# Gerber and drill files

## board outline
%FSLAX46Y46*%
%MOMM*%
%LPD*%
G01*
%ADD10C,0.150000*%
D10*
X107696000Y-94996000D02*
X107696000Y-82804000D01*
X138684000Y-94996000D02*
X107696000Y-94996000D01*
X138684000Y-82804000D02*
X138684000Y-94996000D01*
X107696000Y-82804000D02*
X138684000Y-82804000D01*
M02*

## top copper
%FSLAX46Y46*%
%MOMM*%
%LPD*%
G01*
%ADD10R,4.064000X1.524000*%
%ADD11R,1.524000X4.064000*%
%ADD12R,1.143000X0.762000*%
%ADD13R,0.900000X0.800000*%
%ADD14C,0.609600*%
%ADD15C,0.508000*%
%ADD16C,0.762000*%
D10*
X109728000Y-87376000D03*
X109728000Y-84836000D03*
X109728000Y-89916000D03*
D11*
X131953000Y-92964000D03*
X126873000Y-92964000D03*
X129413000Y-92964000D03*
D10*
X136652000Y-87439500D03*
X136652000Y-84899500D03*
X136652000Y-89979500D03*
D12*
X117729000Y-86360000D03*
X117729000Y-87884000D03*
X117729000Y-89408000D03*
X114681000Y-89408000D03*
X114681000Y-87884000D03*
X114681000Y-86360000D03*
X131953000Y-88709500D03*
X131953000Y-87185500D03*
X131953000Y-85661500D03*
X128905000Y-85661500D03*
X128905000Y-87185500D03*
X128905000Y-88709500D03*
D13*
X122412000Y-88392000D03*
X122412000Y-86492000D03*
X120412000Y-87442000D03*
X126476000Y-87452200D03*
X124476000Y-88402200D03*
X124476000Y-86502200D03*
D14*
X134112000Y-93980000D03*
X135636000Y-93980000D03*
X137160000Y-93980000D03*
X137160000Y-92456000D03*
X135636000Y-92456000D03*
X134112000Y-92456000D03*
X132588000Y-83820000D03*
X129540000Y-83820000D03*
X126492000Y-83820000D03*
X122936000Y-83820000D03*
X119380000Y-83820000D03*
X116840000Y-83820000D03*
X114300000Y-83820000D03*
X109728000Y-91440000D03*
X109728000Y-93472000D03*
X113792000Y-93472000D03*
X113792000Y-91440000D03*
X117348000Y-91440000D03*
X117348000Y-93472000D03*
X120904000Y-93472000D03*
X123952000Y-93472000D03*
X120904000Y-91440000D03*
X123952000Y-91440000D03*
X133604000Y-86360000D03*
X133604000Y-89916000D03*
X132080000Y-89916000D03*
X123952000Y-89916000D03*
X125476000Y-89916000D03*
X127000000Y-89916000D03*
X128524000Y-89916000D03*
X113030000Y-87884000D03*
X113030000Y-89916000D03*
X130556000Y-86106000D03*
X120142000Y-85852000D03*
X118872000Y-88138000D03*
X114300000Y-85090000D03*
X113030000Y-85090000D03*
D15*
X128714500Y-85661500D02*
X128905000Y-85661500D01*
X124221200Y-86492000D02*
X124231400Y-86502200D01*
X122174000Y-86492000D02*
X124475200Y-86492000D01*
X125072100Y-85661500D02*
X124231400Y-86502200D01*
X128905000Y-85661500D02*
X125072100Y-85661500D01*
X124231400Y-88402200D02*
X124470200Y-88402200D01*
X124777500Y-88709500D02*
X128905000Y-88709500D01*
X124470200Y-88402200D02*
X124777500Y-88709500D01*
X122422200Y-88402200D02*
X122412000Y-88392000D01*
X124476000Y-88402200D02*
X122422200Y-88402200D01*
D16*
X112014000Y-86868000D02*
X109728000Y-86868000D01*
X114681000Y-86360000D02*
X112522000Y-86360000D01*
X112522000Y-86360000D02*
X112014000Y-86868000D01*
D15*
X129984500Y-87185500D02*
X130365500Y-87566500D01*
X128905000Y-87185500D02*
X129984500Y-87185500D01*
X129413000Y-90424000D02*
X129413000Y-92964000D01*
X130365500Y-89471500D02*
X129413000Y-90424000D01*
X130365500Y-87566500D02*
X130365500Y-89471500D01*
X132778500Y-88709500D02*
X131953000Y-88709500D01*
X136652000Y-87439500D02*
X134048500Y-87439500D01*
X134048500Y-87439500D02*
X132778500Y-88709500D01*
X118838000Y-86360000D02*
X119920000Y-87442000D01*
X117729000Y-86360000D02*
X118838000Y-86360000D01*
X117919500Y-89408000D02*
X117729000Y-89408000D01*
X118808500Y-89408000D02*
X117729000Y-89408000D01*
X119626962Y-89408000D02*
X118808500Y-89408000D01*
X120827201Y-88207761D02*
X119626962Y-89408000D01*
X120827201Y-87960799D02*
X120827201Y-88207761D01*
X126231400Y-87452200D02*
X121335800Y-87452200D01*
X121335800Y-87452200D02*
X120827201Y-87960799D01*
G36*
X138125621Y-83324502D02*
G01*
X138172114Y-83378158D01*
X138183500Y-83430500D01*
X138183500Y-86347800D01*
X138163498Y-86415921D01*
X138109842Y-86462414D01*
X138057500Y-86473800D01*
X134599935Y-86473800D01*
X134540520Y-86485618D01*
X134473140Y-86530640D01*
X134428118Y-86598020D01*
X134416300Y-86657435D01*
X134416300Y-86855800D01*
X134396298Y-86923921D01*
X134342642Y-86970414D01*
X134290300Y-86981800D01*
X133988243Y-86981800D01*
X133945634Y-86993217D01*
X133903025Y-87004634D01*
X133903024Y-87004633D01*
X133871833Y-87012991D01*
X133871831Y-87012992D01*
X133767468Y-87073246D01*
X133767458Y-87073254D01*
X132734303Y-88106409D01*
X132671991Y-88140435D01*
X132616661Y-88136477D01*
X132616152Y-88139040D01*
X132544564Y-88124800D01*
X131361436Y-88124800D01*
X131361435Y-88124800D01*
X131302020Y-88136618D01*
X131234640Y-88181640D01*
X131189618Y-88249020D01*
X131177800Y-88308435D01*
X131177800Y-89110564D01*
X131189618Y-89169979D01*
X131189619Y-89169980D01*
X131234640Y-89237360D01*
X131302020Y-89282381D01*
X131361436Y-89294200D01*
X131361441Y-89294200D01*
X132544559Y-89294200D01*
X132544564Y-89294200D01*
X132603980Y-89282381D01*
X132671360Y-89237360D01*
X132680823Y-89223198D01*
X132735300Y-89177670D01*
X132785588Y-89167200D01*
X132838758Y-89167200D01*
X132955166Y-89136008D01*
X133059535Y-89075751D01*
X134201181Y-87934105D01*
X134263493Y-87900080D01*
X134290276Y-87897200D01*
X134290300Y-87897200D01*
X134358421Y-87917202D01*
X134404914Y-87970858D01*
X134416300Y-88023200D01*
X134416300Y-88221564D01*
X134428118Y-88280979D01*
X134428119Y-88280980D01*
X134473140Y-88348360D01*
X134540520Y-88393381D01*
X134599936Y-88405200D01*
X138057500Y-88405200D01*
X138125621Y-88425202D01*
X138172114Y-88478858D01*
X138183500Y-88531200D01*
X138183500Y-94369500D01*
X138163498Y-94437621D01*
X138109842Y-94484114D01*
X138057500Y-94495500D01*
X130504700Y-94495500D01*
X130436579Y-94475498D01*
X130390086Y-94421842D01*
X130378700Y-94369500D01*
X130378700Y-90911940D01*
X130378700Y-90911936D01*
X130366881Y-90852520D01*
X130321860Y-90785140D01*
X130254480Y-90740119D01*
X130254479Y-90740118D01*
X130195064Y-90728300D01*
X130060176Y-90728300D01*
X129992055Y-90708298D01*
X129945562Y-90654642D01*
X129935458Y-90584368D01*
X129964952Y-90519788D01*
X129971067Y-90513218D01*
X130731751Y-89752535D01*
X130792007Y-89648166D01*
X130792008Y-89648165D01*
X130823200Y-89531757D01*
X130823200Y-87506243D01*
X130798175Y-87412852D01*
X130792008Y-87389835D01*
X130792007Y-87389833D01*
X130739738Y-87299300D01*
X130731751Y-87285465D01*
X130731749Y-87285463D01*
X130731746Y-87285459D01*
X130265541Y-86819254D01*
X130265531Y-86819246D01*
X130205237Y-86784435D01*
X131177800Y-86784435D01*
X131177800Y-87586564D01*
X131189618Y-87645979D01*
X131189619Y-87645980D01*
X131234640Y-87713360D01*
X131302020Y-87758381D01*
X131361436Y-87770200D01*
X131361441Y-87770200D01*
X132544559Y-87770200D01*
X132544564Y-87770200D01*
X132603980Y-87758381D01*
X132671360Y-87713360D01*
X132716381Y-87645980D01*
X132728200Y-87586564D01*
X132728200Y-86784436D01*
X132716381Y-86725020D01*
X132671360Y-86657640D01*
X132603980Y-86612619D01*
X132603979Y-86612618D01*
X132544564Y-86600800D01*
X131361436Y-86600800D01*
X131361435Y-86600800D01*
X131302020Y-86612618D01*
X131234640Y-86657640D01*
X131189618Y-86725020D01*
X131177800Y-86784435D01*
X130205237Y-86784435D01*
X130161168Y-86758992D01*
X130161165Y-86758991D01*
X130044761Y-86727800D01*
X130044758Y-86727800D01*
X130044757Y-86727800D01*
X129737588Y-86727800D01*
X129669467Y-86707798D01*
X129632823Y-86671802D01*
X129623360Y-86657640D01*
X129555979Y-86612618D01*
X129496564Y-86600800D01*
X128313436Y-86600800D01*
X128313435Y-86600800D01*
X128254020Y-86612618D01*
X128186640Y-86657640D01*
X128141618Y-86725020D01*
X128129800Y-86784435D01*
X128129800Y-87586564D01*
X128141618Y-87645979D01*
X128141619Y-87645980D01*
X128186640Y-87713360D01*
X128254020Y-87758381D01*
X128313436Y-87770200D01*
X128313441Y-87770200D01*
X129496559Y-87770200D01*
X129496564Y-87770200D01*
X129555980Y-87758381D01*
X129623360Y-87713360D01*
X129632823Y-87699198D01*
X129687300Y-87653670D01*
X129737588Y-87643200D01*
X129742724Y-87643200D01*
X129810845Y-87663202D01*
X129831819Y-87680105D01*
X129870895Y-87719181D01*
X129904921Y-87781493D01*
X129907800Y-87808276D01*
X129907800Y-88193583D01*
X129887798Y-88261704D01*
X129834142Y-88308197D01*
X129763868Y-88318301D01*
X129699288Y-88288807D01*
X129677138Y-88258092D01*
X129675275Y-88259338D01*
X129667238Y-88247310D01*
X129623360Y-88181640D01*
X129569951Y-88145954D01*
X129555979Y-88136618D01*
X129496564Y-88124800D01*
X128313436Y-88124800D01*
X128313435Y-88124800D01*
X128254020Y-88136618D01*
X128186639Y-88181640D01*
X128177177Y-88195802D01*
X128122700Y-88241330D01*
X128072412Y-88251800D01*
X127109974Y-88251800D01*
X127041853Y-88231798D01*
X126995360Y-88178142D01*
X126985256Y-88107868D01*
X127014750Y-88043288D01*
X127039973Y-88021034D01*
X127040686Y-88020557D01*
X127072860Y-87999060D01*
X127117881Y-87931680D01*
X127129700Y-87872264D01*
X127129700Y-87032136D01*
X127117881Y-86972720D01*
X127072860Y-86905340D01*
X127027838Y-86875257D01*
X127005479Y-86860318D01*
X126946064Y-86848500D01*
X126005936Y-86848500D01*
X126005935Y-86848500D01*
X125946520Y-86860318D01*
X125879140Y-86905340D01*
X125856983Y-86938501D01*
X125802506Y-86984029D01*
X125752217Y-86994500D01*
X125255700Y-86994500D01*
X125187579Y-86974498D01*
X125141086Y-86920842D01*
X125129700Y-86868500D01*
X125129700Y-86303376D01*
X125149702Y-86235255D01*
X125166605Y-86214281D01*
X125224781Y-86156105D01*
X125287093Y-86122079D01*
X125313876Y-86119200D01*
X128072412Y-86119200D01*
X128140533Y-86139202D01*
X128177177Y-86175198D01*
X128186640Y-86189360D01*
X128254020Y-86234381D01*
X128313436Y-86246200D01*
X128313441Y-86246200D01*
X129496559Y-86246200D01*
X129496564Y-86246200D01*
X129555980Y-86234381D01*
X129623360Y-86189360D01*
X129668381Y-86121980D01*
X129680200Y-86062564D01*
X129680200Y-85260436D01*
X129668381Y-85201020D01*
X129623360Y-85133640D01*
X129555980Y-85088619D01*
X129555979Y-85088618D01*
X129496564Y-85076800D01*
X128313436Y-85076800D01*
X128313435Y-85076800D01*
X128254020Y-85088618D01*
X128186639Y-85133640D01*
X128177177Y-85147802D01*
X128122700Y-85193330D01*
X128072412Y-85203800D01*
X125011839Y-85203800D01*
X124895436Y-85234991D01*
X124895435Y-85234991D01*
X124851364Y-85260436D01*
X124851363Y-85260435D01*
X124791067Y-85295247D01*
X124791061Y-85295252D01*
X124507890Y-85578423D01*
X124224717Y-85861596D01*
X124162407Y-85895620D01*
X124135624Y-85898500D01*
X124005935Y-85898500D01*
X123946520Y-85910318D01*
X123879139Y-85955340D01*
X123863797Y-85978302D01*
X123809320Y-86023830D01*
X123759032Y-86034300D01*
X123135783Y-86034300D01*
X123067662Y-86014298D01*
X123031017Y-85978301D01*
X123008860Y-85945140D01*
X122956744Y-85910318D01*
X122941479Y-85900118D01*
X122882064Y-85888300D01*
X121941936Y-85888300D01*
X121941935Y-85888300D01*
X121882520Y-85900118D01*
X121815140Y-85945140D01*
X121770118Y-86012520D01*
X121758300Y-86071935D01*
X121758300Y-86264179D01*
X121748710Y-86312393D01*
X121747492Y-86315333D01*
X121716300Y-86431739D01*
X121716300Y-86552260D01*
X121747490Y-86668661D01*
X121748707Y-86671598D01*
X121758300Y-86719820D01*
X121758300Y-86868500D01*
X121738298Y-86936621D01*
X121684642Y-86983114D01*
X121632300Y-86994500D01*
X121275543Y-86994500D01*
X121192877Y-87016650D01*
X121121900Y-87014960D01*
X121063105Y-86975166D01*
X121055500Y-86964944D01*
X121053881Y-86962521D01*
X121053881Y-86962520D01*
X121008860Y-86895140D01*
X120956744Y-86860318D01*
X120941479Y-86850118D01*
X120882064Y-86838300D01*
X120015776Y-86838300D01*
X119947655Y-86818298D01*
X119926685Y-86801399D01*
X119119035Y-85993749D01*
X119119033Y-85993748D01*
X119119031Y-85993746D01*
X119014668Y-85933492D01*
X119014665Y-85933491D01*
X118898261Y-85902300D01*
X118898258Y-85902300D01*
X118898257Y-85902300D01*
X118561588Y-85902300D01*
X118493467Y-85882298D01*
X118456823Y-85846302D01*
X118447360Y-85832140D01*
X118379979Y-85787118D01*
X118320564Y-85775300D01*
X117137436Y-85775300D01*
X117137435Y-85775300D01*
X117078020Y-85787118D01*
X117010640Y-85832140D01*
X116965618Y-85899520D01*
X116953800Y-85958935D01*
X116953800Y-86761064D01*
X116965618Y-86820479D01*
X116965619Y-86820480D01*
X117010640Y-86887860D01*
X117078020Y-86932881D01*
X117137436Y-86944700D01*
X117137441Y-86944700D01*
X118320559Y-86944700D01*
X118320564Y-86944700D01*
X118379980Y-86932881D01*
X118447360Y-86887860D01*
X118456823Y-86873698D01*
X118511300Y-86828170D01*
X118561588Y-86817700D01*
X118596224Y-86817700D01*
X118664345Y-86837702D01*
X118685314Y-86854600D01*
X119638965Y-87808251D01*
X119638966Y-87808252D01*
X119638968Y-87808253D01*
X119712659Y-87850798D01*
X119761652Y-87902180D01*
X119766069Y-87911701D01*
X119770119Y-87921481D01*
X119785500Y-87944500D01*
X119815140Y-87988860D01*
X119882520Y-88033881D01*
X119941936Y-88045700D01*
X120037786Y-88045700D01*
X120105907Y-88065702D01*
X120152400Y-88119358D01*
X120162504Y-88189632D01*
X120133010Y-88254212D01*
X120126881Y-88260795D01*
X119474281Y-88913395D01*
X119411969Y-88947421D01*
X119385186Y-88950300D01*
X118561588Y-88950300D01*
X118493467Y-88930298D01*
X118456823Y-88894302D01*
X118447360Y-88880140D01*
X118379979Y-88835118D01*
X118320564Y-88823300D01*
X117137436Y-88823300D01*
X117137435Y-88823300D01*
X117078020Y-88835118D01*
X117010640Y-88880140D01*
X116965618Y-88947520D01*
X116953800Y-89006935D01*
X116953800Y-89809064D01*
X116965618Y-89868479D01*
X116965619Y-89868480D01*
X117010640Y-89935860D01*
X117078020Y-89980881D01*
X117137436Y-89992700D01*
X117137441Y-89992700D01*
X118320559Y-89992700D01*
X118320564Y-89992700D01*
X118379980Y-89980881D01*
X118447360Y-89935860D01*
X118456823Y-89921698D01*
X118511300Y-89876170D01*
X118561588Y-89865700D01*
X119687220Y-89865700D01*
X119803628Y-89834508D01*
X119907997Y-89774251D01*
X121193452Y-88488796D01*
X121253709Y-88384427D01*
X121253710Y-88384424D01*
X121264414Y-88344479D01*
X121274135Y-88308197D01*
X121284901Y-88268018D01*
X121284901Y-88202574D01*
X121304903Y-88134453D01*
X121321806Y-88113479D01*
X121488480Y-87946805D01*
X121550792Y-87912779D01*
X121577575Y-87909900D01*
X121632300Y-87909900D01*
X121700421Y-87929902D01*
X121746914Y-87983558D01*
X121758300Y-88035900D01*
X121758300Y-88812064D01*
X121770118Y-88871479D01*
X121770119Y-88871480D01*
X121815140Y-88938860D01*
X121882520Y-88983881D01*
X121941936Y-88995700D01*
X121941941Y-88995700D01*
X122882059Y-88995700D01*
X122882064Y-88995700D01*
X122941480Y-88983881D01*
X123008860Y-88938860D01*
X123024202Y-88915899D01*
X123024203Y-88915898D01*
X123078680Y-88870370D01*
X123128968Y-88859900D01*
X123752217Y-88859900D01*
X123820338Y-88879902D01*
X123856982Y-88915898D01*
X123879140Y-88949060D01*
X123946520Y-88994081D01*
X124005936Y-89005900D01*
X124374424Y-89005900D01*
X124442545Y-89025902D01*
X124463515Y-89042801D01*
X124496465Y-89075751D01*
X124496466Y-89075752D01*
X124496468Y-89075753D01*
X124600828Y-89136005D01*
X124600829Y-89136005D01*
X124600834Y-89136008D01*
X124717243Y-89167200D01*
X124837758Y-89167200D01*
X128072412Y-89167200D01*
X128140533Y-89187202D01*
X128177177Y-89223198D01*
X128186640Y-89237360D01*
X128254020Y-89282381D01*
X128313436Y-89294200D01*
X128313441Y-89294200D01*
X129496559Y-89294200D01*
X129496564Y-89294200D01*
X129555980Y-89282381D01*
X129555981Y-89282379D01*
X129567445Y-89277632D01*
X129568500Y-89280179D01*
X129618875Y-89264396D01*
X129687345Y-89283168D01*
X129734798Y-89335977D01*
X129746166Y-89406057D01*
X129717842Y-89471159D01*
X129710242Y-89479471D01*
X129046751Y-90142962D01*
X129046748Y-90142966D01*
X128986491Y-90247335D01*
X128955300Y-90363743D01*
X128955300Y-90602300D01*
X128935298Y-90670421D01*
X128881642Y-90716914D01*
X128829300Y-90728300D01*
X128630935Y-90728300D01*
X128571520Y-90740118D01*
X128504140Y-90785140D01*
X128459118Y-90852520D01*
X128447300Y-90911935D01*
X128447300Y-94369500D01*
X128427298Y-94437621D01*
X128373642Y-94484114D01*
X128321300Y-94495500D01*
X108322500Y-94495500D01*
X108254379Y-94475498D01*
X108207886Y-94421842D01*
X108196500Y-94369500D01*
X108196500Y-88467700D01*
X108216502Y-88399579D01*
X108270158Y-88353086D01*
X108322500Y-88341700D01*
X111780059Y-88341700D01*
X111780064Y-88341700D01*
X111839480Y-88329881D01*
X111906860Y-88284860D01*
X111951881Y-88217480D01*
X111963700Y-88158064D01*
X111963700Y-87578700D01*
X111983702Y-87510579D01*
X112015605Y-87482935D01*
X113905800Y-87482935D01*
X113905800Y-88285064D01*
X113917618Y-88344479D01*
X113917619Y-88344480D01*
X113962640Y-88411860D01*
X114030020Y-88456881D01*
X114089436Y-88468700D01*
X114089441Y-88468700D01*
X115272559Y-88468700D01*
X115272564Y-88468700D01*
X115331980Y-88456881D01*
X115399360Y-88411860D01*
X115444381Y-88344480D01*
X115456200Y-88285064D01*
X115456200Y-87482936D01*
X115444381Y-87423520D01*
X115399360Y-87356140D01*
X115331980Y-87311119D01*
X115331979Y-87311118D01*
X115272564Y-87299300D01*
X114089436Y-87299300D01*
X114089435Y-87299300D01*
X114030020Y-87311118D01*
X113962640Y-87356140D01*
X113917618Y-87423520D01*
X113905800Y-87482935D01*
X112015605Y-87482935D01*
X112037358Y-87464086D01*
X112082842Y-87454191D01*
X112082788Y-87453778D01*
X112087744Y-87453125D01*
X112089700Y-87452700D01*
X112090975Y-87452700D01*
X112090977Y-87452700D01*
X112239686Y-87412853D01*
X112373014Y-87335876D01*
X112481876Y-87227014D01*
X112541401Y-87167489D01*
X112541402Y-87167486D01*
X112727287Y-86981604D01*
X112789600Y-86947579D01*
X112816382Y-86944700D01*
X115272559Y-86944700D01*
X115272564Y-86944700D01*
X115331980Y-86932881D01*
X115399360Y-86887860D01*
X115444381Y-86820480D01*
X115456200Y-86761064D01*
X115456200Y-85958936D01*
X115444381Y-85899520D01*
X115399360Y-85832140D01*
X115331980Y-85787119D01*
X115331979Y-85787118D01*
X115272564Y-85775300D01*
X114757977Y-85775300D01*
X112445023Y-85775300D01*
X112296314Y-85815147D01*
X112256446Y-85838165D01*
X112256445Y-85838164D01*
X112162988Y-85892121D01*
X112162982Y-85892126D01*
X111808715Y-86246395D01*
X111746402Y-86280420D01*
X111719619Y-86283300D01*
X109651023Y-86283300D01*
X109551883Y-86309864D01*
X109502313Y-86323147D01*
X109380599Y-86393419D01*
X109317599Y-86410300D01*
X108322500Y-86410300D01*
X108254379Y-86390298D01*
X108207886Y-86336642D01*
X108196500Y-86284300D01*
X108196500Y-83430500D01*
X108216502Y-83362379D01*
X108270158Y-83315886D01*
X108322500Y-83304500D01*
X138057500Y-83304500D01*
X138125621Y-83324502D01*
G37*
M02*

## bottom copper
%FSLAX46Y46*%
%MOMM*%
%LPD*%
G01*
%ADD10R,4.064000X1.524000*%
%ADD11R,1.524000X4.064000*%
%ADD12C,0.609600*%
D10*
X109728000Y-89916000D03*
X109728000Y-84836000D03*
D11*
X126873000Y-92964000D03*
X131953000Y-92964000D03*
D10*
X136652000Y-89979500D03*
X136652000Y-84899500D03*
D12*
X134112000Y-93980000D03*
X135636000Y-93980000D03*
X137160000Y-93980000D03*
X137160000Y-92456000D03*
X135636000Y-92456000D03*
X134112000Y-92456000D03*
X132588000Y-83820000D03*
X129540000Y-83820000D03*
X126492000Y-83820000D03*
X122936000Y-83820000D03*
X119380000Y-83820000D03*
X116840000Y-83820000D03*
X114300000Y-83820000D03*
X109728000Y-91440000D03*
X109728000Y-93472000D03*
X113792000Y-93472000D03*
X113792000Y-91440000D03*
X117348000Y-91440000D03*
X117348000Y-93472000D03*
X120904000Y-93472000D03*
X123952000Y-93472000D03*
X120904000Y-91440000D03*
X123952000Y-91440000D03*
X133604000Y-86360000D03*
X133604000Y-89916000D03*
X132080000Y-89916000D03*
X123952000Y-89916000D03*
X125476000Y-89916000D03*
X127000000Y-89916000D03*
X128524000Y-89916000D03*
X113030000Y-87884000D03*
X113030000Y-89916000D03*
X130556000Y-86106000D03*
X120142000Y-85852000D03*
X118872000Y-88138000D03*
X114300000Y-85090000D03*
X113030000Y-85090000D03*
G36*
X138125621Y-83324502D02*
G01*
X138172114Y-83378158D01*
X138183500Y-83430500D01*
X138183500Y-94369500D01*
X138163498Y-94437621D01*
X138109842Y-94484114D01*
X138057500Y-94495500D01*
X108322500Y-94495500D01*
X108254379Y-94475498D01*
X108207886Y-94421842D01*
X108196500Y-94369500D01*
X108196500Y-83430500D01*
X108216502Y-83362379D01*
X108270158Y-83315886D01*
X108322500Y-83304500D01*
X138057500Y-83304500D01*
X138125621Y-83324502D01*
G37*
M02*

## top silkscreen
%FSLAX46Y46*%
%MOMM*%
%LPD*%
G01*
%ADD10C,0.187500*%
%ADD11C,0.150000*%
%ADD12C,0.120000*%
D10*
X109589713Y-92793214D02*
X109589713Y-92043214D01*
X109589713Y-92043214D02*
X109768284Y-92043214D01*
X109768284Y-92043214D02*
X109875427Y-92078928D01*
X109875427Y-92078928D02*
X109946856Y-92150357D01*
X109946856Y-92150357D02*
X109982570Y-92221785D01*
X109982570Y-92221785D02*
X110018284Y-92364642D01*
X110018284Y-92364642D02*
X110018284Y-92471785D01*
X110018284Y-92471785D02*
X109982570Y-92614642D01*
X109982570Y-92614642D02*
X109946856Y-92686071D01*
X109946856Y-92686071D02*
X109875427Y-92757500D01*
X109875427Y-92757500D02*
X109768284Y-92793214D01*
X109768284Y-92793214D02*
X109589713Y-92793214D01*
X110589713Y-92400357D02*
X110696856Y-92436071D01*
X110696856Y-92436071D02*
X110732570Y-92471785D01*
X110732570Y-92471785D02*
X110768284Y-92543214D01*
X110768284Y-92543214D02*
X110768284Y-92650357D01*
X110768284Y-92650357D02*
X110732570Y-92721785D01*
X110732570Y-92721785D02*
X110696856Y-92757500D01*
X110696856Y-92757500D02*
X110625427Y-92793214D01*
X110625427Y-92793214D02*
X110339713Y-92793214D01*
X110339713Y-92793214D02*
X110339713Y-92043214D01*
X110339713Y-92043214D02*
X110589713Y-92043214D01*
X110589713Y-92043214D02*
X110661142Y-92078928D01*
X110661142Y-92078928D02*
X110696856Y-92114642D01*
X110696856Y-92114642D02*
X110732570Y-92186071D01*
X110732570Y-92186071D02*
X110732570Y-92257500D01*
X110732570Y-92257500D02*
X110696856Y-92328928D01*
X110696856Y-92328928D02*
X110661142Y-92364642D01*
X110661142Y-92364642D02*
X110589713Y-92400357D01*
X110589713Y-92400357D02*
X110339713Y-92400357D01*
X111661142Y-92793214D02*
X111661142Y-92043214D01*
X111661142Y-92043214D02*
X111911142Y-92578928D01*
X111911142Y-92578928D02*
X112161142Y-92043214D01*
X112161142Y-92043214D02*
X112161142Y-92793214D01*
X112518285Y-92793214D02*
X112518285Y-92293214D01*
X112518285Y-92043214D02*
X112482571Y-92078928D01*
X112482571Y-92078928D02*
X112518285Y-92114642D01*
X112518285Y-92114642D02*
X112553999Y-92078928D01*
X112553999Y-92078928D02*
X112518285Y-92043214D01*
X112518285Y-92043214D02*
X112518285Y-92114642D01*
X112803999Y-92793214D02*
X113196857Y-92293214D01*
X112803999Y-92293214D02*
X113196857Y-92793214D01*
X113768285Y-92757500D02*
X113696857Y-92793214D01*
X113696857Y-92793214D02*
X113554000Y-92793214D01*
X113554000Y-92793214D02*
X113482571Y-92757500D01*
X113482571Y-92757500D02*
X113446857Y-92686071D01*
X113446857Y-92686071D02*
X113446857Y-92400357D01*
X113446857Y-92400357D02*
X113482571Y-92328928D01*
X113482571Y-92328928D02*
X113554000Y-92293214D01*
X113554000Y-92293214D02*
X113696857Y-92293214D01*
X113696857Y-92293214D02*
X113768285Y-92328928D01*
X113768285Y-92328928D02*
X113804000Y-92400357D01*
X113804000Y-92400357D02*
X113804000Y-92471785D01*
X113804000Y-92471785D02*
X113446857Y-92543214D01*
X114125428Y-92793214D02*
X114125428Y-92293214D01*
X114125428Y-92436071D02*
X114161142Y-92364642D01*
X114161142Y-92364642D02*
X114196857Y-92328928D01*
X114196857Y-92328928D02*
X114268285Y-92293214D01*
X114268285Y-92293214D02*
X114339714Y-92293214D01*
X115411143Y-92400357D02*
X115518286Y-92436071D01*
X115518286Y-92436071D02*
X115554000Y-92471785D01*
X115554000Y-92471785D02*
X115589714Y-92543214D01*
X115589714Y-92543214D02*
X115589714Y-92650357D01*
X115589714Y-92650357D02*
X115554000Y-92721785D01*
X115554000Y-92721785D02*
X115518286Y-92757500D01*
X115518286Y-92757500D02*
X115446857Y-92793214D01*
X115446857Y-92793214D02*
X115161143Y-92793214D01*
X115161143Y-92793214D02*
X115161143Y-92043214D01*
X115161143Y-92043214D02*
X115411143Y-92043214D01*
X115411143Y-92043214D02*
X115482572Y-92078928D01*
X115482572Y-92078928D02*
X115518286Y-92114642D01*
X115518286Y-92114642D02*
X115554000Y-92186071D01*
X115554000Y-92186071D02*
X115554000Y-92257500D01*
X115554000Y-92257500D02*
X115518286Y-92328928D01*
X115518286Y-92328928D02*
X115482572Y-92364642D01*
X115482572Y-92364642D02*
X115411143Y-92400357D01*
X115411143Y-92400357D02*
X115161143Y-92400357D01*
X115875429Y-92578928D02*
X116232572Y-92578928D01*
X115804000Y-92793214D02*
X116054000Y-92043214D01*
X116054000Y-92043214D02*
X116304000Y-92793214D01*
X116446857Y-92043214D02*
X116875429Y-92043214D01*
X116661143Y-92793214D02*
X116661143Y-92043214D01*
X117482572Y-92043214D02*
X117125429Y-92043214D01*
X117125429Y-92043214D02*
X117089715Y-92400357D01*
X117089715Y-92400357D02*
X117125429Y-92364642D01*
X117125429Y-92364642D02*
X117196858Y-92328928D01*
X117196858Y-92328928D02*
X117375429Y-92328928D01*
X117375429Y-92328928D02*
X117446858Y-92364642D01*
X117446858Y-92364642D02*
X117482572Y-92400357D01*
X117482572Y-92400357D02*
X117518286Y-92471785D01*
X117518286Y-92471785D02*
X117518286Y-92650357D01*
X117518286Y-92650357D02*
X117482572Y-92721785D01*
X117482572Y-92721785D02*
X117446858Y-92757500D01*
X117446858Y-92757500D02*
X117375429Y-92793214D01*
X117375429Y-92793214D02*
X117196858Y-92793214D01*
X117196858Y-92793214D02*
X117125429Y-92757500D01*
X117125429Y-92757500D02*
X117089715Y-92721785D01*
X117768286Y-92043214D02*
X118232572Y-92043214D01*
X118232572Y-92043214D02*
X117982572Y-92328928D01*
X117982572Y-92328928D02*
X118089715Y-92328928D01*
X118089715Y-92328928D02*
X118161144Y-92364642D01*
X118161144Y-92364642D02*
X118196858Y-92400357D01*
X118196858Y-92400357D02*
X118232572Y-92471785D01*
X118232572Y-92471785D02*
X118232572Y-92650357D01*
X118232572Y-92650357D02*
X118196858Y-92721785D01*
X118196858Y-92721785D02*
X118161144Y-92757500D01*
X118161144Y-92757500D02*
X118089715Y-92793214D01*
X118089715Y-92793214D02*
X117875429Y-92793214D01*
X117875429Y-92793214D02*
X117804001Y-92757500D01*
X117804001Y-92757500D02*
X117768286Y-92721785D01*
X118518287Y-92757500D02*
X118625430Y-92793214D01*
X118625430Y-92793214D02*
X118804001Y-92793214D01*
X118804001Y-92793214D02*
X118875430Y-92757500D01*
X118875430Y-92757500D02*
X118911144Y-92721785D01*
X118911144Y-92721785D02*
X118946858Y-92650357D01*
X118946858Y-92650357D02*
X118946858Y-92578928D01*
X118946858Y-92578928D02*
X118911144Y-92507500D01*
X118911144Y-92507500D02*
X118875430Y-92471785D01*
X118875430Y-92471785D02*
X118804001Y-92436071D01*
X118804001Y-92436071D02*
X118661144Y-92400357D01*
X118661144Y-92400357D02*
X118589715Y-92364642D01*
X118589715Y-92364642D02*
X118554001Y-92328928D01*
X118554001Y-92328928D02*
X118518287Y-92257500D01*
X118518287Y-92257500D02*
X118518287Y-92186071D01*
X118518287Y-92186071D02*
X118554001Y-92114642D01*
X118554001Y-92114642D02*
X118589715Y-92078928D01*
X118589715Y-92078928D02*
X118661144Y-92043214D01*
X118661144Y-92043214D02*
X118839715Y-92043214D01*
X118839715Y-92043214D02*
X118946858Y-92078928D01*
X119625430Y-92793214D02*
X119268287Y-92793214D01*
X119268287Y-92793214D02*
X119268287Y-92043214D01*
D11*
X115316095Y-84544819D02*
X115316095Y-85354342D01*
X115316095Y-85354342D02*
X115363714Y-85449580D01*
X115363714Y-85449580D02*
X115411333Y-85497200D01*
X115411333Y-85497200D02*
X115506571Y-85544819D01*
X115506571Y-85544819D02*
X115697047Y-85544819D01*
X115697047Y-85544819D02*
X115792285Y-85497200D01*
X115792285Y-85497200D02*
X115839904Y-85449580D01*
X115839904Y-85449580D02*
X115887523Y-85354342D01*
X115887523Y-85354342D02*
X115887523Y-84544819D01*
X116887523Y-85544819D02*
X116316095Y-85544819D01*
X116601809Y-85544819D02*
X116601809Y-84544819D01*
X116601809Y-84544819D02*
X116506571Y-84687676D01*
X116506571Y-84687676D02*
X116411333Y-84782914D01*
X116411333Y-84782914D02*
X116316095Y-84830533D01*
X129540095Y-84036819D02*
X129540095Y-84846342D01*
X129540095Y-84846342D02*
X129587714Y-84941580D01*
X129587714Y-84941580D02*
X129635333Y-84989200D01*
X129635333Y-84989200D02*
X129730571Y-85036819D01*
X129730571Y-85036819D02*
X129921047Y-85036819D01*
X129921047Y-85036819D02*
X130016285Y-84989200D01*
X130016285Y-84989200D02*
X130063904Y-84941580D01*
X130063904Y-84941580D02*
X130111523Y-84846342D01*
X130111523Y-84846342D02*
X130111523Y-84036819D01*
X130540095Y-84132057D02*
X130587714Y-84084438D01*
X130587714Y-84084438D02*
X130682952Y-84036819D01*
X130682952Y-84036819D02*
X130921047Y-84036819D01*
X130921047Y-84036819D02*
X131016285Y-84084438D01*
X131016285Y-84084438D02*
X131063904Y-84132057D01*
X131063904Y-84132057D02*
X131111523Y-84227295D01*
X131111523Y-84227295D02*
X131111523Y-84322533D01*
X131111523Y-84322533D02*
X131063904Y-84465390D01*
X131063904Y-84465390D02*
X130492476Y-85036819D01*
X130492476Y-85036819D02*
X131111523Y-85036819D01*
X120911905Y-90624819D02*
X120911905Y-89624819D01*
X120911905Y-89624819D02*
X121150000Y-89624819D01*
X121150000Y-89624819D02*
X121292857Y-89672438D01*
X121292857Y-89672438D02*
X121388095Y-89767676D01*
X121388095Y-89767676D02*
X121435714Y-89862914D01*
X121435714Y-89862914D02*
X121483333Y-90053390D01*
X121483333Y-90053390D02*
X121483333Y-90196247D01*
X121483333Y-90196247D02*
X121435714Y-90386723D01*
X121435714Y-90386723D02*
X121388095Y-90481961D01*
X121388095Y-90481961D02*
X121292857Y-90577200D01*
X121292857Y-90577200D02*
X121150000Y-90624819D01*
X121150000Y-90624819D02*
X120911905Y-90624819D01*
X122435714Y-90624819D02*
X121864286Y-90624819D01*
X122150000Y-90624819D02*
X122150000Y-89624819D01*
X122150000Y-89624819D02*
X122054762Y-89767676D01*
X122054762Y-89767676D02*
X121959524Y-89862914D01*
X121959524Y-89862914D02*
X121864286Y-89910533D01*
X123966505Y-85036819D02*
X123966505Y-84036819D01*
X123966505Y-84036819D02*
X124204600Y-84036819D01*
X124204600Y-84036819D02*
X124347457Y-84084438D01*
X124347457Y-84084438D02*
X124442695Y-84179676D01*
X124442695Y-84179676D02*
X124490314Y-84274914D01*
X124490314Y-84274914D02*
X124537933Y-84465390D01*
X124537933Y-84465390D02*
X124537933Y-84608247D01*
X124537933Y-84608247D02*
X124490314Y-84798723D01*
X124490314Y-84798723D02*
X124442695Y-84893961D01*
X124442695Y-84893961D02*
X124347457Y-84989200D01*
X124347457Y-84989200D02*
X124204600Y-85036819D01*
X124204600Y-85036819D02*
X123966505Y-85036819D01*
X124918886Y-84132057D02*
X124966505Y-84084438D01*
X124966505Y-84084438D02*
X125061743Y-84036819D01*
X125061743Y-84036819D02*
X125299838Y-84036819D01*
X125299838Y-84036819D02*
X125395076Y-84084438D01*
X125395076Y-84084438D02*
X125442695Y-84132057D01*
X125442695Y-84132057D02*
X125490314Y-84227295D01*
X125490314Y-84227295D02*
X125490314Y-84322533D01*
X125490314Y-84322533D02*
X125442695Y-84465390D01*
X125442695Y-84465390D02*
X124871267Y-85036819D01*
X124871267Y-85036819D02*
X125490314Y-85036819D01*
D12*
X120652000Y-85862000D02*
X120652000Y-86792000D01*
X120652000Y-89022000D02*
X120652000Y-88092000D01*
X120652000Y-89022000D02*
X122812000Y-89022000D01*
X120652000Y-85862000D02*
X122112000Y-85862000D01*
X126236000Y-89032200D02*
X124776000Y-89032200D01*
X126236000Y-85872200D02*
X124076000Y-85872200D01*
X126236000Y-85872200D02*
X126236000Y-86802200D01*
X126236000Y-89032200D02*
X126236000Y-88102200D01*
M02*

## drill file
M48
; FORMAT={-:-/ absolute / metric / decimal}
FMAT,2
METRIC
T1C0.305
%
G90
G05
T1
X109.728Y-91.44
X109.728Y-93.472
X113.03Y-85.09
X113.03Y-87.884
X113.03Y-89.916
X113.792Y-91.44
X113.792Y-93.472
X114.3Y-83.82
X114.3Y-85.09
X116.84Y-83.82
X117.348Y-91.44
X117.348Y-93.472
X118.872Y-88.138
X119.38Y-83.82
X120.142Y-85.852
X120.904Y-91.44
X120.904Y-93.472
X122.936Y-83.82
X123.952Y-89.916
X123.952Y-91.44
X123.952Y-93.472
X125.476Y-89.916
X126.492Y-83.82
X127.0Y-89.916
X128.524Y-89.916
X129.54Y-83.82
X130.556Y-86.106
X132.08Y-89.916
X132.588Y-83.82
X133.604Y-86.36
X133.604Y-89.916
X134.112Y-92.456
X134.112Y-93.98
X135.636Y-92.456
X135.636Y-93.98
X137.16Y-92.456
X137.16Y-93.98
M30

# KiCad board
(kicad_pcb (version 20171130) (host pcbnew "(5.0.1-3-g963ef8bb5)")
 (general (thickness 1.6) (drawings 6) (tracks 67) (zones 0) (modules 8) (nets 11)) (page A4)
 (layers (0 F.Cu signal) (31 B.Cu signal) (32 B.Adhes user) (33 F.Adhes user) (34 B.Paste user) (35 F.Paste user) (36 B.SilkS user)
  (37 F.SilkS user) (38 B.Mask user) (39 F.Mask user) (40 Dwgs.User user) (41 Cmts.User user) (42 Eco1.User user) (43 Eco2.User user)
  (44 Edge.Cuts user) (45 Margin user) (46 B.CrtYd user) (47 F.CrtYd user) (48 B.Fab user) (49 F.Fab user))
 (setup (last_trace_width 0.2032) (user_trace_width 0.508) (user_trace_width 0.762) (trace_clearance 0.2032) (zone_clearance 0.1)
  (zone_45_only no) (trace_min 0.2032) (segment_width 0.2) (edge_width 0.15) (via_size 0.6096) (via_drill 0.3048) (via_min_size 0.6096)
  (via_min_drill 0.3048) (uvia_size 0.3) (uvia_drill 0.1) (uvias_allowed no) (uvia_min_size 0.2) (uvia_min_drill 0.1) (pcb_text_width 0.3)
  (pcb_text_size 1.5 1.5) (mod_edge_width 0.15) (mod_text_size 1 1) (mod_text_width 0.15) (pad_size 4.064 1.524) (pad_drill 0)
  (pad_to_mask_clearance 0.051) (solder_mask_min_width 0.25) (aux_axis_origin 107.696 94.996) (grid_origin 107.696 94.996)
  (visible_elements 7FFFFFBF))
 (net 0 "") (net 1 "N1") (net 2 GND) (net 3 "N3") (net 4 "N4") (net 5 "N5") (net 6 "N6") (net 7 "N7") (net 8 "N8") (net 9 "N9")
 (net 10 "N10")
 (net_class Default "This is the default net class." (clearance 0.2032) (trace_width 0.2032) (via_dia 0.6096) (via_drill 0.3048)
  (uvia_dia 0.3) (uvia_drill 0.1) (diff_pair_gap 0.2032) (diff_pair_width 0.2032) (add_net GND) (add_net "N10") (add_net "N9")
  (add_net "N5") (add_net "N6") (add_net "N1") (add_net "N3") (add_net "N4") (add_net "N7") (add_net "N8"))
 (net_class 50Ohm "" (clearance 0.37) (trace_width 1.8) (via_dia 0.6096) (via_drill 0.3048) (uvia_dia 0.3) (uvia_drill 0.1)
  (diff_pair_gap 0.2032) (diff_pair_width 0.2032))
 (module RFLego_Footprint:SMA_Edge (layer F.Cu) (at 107.696 87.376)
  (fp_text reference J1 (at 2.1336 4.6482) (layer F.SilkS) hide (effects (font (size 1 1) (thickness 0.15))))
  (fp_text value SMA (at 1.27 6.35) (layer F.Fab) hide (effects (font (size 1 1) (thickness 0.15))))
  (pad 1 smd rect (at 2.032 0) (size 4.064 1.524) (layers F.Cu F.Mask) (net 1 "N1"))
  (pad 2 smd rect (at 2.032 -2.54) (size 4.064 1.524) (layers F.Cu F.Mask) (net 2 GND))
  (pad 2 smd rect (at 2.032 2.54) (size 4.064 1.524) (layers B.Cu B.Mask) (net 2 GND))
  (pad 2 smd rect (at 2.032 -2.54) (size 4.064 1.524) (layers B.Cu B.Mask) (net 2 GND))
  (pad 2 smd rect (at 2.032 2.54) (size 4.064 1.524) (layers F.Cu F.Mask) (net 2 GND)))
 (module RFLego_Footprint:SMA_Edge (layer F.Cu) (at 129.413 94.996 90)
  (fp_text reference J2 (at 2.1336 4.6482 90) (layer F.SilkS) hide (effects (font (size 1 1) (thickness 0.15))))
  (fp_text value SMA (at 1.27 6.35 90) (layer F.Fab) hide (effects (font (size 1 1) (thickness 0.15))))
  (pad 2 smd rect (at 2.032 2.54 90) (size 4.064 1.524) (layers F.Cu F.Mask) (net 2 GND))
  (pad 2 smd rect (at 2.032 -2.54 90) (size 4.064 1.524) (layers B.Cu B.Mask) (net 2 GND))
  (pad 2 smd rect (at 2.032 2.54 90) (size 4.064 1.524) (layers B.Cu B.Mask) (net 2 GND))
  (pad 2 smd rect (at 2.032 -2.54 90) (size 4.064 1.524) (layers F.Cu F.Mask) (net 2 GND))
  (pad 1 smd rect (at 2.032 0 90) (size 4.064 1.524) (layers F.Cu F.Mask) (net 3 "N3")))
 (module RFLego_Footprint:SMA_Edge (layer F.Cu) (at 134.62 87.4395)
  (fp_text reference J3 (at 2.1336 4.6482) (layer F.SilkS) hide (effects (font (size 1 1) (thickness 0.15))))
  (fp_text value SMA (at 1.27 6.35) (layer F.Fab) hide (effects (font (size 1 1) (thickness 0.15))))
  (pad 1 smd rect (at 2.032 0) (size 4.064 1.524) (layers F.Cu F.Mask) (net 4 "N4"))
  (pad 2 smd rect (at 2.032 -2.54) (size 4.064 1.524) (layers F.Cu F.Mask) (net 2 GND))
  (pad 2 smd rect (at 2.032 2.54) (size 4.064 1.524) (layers B.Cu B.Mask) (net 2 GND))
  (pad 2 smd rect (at 2.032 -2.54) (size 4.064 1.524) (layers B.Cu B.Mask) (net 2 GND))
  (pad 2 smd rect (at 2.032 2.54) (size 4.064 1.524) (layers F.Cu F.Mask) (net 2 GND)))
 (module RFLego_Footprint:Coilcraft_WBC (layer F.Cu) (at 117.729 86.36 270)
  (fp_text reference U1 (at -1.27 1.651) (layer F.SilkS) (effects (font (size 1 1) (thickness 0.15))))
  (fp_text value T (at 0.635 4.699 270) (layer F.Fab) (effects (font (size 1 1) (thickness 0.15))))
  (pad 1 smd rect (at 0 0 270) (size 0.762 1.143) (layers F.Cu F.Paste F.Mask) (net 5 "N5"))
  (pad 2 smd rect (at 1.524 0 270) (size 0.762 1.143) (layers F.Cu F.Paste F.Mask) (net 2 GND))
  (pad 3 smd rect (at 3.048 0 270) (size 0.762 1.143) (layers F.Cu F.Paste F.Mask) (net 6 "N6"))
  (pad 4 smd rect (at 3.048 3.048 270) (size 0.762 1.143) (layers F.Cu F.Paste F.Mask) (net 2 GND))
  (pad 5 smd rect (at 1.524 3.048 270) (size 0.762 1.143) (layers F.Cu F.Paste F.Mask) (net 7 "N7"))
  (pad 6 smd rect (at 0 3.048 270) (size 0.762 1.143) (layers F.Cu F.Paste F.Mask) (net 1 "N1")))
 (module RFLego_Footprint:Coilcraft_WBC (layer F.Cu) (at 128.905 88.7095 90)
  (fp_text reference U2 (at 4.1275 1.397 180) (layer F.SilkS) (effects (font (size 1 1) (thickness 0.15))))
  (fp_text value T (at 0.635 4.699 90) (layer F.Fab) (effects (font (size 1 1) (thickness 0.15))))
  (pad 6 smd rect (at 0 3.048 90) (size 0.762 1.143) (layers F.Cu F.Paste F.Mask) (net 4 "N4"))
  (pad 5 smd rect (at 1.524 3.048 90) (size 0.762 1.143) (layers F.Cu F.Paste F.Mask) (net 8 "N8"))
  (pad 4 smd rect (at 3.048 3.048 90) (size 0.762 1.143) (layers F.Cu F.Paste F.Mask) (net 2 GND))
  (pad 3 smd rect (at 3.048 0 90) (size 0.762 1.143) (layers F.Cu F.Paste F.Mask) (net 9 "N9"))
  (pad 2 smd rect (at 1.524 0 90) (size 0.762 1.143) (layers F.Cu F.Paste F.Mask) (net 3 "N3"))
  (pad 1 smd rect (at 0 0 90) (size 0.762 1.143) (layers F.Cu F.Paste F.Mask) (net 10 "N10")))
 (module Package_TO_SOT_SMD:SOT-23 (layer F.Cu) (at 121.412 87.442 180)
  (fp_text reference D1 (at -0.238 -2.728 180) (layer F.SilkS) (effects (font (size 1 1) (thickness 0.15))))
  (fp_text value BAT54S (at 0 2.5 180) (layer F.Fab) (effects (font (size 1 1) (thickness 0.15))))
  (fp_line (start 0.76 1.58) (end 0.76 0.65) (layer F.SilkS) (width 0.12))
  (fp_line (start 0.76 -1.58) (end 0.76 -0.65) (layer F.SilkS) (width 0.12))
  (fp_line (start 0.76 -1.58) (end -1.4 -1.58) (layer F.SilkS) (width 0.12))
  (fp_line (start 0.76 1.58) (end -0.7 1.58) (layer F.SilkS) (width 0.12))
  (pad 1 smd rect (at -1 -0.95 180) (size 0.9 0.8) (layers F.Cu F.Paste F.Mask) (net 10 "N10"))
  (pad 2 smd rect (at -1 0.95 180) (size 0.9 0.8) (layers F.Cu F.Paste F.Mask) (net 9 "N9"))
  (pad 3 smd rect (at 1 0 180) (size 0.9 0.8) (layers F.Cu F.Paste F.Mask) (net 5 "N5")))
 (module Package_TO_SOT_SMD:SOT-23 (layer F.Cu) (at 125.476 87.4522)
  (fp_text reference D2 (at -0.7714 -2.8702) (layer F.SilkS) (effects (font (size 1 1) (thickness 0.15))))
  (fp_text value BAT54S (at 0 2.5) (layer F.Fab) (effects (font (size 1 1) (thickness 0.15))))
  (fp_line (start 0.76 1.58) (end -0.7 1.58) (layer F.SilkS) (width 0.12))
  (fp_line (start 0.76 -1.58) (end -1.4 -1.58) (layer F.SilkS) (width 0.12))
  (fp_line (start 0.76 -1.58) (end 0.76 -0.65) (layer F.SilkS) (width 0.12))
  (fp_line (start 0.76 1.58) (end 0.76 0.65) (layer F.SilkS) (width 0.12))
  (pad 3 smd rect (at 1 0) (size 0.9 0.8) (layers F.Cu F.Paste F.Mask) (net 6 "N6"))
  (pad 2 smd rect (at -1 0.95) (size 0.9 0.8) (layers F.Cu F.Paste F.Mask) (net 10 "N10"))
  (pad 1 smd rect (at -1 -0.95) (size 0.9 0.8) (layers F.Cu F.Paste F.Mask) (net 9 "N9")))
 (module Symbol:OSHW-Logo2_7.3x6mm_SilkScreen (layer B.Cu) (at 129.54 86.868 180)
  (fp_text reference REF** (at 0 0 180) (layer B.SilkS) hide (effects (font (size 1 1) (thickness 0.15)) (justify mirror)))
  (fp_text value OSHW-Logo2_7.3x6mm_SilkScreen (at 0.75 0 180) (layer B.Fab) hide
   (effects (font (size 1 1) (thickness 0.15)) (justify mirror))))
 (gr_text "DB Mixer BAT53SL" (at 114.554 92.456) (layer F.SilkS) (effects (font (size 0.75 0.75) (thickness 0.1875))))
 (gr_line (start 107.696 94.996) (end 107.696 82.804) (layer Edge.Cuts) (width 0.15))
 (gr_line (start 138.684 94.996) (end 107.696 94.996) (layer Edge.Cuts) (width 0.15))
 (gr_line (start 138.684 82.804) (end 138.684 94.996) (layer Edge.Cuts) (width 0.15))
 (gr_line (start 107.696 82.804) (end 138.684 82.804) (layer Edge.Cuts) (width 0.15))
 (segment (start 128.7145 85.6615) (end 128.905 85.6615) (width 0.508) (layer F.Cu) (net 9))
 (segment (start 124.2212 86.492) (end 124.2314 86.5022) (width 0.508) (layer F.Cu) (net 9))
 (segment (start 122.174 86.492) (end 124.4752 86.492) (width 0.508) (layer F.Cu) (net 9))
 (segment (start 125.0721 85.6615) (end 124.2314 86.5022) (width 0.508) (layer F.Cu) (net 9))
 (segment (start 128.905 85.6615) (end 125.0721 85.6615) (width 0.508) (layer F.Cu) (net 9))
 (segment (start 124.2314 88.4022) (end 124.4702 88.4022) (width 0.508) (layer F.Cu) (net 10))
 (segment (start 124.7775 88.7095) (end 128.905 88.7095) (width 0.508) (layer F.Cu) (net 10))
 (segment (start 124.4702 88.4022) (end 124.7775 88.7095) (width 0.508) (layer F.Cu) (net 10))
 (segment (start 122.4222 88.4022) (end 122.412 88.392) (width 0.508) (layer F.Cu) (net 10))
 (segment (start 124.476 88.4022) (end 122.4222 88.4022) (width 0.508) (layer F.Cu) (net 10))
 (segment (start 112.014 86.868) (end 109.728 86.868) (width 0.762) (layer F.Cu) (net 1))
 (segment (start 114.681 86.36) (end 112.522 86.36) (width 0.762) (layer F.Cu) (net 1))
 (segment (start 112.522 86.36) (end 112.014 86.868) (width 0.762) (layer F.Cu) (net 1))
 (via (at 134.112 93.98) (size 0.6096) (drill 0.3048) (layers F.Cu B.Cu) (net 2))
 (via (at 135.636 93.98) (size 0.6096) (drill 0.3048) (layers F.Cu B.Cu) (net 2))
 (via (at 137.16 93.98) (size 0.6096) (drill 0.3048) (layers F.Cu B.Cu) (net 2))
 (via (at 137.16 92.456) (size 0.6096) (drill 0.3048) (layers F.Cu B.Cu) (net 2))
 (via (at 135.636 92.456) (size 0.6096) (drill 0.3048) (layers F.Cu B.Cu) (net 2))
 (via (at 134.112 92.456) (size 0.6096) (drill 0.3048) (layers F.Cu B.Cu) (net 2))
 (via (at 132.588 83.82) (size 0.6096) (drill 0.3048) (layers F.Cu B.Cu) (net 2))
 (via (at 129.54 83.82) (size 0.6096) (drill 0.3048) (layers F.Cu B.Cu) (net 2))
 (via (at 126.492 83.82) (size 0.6096) (drill 0.3048) (layers F.Cu B.Cu) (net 2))
 (via (at 122.936 83.82) (size 0.6096) (drill 0.3048) (layers F.Cu B.Cu) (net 2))
 (via (at 119.38 83.82) (size 0.6096) (drill 0.3048) (layers F.Cu B.Cu) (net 2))
 (via (at 116.84 83.82) (size 0.6096) (drill 0.3048) (layers F.Cu B.Cu) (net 2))
 (via (at 114.3 83.82) (size 0.6096) (drill 0.3048) (layers F.Cu B.Cu) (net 2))
 (via (at 109.728 91.44) (size 0.6096) (drill 0.3048) (layers F.Cu B.Cu) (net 2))
 (via (at 109.728 93.472) (size 0.6096) (drill 0.3048) (layers F.Cu B.Cu) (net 2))
 (via (at 113.792 93.472) (size 0.6096) (drill 0.3048) (layers F.Cu B.Cu) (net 2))
 (via (at 113.792 91.44) (size 0.6096) (drill 0.3048) (layers F.Cu B.Cu) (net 2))
 (via (at 117.348 91.44) (size 0.6096) (drill 0.3048) (layers F.Cu B.Cu) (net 2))
 (via (at 117.348 93.472) (size 0.6096) (drill 0.3048) (layers F.Cu B.Cu) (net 2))
 (via (at 120.904 93.472) (size 0.6096) (drill 0.3048) (layers F.Cu B.Cu) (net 2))
 (via (at 123.952 93.472) (size 0.6096) (drill 0.3048) (layers F.Cu B.Cu) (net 2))
 (via (at 120.904 91.44) (size 0.6096) (drill 0.3048) (layers F.Cu B.Cu) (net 2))
 (via (at 123.952 91.44) (size 0.6096) (drill 0.3048) (layers F.Cu B.Cu) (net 2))
 (via (at 133.604 86.36) (size 0.6096) (drill 0.3048) (layers F.Cu B.Cu) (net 2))
 (via (at 133.604 89.916) (size 0.6096) (drill 0.3048) (layers F.Cu B.Cu) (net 2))
 (via (at 132.08 89.916) (size 0.6096) (drill 0.3048) (layers F.Cu B.Cu) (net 2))
 (via (at 123.952 89.916) (size 0.6096) (drill 0.3048) (layers F.Cu B.Cu) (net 2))
 (via (at 125.476 89.916) (size 0.6096) (drill 0.3048) (layers F.Cu B.Cu) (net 2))
 (via (at 127 89.916) (size 0.6096) (drill 0.3048) (layers F.Cu B.Cu) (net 2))
 (via (at 128.524 89.916) (size 0.6096) (drill 0.3048) (layers F.Cu B.Cu) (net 2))
 (via (at 113.03 87.884) (size 0.6096) (drill 0.3048) (layers F.Cu B.Cu) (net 2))
 (via (at 113.03 89.916) (size 0.6096) (drill 0.3048) (layers F.Cu B.Cu) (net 2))
 (via (at 130.556 86.106) (size 0.6096) (drill 0.3048) (layers F.Cu B.Cu) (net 2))
 (via (at 120.142 85.852) (size 0.6096) (drill 0.3048) (layers F.Cu B.Cu) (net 2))
 (via (at 118.872 88.138) (size 0.6096) (drill 0.3048) (layers F.Cu B.Cu) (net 2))
 (via (at 114.3 85.09) (size 0.6096) (drill 0.3048) (layers F.Cu B.Cu) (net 2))
 (via (at 113.03 85.09) (size 0.6096) (drill 0.3048) (layers F.Cu B.Cu) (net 2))
 (segment (start 129.9845 87.1855) (end 130.3655 87.5665) (width 0.508) (layer F.Cu) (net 3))
 (segment (start 128.905 87.1855) (end 129.9845 87.1855) (width 0.508) (layer F.Cu) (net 3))
 (segment (start 129.413 90.424) (end 129.413 92.964) (width 0.508) (layer F.Cu) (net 3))
 (segment (start 130.3655 89.4715) (end 129.413 90.424) (width 0.508) (layer F.Cu) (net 3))
 (segment (start 130.3655 87.5665) (end 130.3655 89.4715) (width 0.508) (layer F.Cu) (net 3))
 (segment (start 132.7785 88.7095) (end 131.953 88.7095) (width 0.508) (layer F.Cu) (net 4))
 (segment (start 136.652 87.4395) (end 134.0485 87.4395) (width 0.508) (layer F.Cu) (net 4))
 (segment (start 134.0485 87.4395) (end 132.7785 88.7095) (width 0.508) (layer F.Cu) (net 4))
 (segment (start 118.838 86.36) (end 119.92 87.442) (width 0.508) (layer F.Cu) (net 5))
 (segment (start 117.729 86.36) (end 118.838 86.36) (width 0.508) (layer F.Cu) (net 5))
 (segment (start 117.9195 89.408) (end 117.729 89.408) (width 0.508) (layer F.Cu) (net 6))
 (segment (start 118.8085 89.408) (end 117.729 89.408) (width 0.508) (layer F.Cu) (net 6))
 (segment (start 119.626962 89.408) (end 118.8085 89.408) (width 0.508) (layer F.Cu) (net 6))
 (segment (start 120.827201 88.207761) (end 119.626962 89.408) (width 0.508) (layer F.Cu) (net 6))
 (segment (start 120.827201 87.960799) (end 120.827201 88.207761) (width 0.508) (layer F.Cu) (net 6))
 (segment (start 126.2314 87.4522) (end 121.3358 87.4522) (width 0.508) (layer F.Cu) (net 6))
 (segment (start 121.3358 87.4522) (end 120.827201 87.960799) (width 0.508) (layer F.Cu) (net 6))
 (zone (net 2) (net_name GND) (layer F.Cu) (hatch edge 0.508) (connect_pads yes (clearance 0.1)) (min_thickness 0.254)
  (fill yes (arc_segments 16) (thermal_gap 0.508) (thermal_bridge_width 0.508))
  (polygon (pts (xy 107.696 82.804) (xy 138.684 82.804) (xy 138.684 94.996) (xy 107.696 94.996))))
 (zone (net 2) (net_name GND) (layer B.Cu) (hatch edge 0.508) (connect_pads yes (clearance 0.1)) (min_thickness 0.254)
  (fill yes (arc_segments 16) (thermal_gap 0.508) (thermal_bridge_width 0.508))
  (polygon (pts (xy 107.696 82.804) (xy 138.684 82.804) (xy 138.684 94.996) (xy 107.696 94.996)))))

